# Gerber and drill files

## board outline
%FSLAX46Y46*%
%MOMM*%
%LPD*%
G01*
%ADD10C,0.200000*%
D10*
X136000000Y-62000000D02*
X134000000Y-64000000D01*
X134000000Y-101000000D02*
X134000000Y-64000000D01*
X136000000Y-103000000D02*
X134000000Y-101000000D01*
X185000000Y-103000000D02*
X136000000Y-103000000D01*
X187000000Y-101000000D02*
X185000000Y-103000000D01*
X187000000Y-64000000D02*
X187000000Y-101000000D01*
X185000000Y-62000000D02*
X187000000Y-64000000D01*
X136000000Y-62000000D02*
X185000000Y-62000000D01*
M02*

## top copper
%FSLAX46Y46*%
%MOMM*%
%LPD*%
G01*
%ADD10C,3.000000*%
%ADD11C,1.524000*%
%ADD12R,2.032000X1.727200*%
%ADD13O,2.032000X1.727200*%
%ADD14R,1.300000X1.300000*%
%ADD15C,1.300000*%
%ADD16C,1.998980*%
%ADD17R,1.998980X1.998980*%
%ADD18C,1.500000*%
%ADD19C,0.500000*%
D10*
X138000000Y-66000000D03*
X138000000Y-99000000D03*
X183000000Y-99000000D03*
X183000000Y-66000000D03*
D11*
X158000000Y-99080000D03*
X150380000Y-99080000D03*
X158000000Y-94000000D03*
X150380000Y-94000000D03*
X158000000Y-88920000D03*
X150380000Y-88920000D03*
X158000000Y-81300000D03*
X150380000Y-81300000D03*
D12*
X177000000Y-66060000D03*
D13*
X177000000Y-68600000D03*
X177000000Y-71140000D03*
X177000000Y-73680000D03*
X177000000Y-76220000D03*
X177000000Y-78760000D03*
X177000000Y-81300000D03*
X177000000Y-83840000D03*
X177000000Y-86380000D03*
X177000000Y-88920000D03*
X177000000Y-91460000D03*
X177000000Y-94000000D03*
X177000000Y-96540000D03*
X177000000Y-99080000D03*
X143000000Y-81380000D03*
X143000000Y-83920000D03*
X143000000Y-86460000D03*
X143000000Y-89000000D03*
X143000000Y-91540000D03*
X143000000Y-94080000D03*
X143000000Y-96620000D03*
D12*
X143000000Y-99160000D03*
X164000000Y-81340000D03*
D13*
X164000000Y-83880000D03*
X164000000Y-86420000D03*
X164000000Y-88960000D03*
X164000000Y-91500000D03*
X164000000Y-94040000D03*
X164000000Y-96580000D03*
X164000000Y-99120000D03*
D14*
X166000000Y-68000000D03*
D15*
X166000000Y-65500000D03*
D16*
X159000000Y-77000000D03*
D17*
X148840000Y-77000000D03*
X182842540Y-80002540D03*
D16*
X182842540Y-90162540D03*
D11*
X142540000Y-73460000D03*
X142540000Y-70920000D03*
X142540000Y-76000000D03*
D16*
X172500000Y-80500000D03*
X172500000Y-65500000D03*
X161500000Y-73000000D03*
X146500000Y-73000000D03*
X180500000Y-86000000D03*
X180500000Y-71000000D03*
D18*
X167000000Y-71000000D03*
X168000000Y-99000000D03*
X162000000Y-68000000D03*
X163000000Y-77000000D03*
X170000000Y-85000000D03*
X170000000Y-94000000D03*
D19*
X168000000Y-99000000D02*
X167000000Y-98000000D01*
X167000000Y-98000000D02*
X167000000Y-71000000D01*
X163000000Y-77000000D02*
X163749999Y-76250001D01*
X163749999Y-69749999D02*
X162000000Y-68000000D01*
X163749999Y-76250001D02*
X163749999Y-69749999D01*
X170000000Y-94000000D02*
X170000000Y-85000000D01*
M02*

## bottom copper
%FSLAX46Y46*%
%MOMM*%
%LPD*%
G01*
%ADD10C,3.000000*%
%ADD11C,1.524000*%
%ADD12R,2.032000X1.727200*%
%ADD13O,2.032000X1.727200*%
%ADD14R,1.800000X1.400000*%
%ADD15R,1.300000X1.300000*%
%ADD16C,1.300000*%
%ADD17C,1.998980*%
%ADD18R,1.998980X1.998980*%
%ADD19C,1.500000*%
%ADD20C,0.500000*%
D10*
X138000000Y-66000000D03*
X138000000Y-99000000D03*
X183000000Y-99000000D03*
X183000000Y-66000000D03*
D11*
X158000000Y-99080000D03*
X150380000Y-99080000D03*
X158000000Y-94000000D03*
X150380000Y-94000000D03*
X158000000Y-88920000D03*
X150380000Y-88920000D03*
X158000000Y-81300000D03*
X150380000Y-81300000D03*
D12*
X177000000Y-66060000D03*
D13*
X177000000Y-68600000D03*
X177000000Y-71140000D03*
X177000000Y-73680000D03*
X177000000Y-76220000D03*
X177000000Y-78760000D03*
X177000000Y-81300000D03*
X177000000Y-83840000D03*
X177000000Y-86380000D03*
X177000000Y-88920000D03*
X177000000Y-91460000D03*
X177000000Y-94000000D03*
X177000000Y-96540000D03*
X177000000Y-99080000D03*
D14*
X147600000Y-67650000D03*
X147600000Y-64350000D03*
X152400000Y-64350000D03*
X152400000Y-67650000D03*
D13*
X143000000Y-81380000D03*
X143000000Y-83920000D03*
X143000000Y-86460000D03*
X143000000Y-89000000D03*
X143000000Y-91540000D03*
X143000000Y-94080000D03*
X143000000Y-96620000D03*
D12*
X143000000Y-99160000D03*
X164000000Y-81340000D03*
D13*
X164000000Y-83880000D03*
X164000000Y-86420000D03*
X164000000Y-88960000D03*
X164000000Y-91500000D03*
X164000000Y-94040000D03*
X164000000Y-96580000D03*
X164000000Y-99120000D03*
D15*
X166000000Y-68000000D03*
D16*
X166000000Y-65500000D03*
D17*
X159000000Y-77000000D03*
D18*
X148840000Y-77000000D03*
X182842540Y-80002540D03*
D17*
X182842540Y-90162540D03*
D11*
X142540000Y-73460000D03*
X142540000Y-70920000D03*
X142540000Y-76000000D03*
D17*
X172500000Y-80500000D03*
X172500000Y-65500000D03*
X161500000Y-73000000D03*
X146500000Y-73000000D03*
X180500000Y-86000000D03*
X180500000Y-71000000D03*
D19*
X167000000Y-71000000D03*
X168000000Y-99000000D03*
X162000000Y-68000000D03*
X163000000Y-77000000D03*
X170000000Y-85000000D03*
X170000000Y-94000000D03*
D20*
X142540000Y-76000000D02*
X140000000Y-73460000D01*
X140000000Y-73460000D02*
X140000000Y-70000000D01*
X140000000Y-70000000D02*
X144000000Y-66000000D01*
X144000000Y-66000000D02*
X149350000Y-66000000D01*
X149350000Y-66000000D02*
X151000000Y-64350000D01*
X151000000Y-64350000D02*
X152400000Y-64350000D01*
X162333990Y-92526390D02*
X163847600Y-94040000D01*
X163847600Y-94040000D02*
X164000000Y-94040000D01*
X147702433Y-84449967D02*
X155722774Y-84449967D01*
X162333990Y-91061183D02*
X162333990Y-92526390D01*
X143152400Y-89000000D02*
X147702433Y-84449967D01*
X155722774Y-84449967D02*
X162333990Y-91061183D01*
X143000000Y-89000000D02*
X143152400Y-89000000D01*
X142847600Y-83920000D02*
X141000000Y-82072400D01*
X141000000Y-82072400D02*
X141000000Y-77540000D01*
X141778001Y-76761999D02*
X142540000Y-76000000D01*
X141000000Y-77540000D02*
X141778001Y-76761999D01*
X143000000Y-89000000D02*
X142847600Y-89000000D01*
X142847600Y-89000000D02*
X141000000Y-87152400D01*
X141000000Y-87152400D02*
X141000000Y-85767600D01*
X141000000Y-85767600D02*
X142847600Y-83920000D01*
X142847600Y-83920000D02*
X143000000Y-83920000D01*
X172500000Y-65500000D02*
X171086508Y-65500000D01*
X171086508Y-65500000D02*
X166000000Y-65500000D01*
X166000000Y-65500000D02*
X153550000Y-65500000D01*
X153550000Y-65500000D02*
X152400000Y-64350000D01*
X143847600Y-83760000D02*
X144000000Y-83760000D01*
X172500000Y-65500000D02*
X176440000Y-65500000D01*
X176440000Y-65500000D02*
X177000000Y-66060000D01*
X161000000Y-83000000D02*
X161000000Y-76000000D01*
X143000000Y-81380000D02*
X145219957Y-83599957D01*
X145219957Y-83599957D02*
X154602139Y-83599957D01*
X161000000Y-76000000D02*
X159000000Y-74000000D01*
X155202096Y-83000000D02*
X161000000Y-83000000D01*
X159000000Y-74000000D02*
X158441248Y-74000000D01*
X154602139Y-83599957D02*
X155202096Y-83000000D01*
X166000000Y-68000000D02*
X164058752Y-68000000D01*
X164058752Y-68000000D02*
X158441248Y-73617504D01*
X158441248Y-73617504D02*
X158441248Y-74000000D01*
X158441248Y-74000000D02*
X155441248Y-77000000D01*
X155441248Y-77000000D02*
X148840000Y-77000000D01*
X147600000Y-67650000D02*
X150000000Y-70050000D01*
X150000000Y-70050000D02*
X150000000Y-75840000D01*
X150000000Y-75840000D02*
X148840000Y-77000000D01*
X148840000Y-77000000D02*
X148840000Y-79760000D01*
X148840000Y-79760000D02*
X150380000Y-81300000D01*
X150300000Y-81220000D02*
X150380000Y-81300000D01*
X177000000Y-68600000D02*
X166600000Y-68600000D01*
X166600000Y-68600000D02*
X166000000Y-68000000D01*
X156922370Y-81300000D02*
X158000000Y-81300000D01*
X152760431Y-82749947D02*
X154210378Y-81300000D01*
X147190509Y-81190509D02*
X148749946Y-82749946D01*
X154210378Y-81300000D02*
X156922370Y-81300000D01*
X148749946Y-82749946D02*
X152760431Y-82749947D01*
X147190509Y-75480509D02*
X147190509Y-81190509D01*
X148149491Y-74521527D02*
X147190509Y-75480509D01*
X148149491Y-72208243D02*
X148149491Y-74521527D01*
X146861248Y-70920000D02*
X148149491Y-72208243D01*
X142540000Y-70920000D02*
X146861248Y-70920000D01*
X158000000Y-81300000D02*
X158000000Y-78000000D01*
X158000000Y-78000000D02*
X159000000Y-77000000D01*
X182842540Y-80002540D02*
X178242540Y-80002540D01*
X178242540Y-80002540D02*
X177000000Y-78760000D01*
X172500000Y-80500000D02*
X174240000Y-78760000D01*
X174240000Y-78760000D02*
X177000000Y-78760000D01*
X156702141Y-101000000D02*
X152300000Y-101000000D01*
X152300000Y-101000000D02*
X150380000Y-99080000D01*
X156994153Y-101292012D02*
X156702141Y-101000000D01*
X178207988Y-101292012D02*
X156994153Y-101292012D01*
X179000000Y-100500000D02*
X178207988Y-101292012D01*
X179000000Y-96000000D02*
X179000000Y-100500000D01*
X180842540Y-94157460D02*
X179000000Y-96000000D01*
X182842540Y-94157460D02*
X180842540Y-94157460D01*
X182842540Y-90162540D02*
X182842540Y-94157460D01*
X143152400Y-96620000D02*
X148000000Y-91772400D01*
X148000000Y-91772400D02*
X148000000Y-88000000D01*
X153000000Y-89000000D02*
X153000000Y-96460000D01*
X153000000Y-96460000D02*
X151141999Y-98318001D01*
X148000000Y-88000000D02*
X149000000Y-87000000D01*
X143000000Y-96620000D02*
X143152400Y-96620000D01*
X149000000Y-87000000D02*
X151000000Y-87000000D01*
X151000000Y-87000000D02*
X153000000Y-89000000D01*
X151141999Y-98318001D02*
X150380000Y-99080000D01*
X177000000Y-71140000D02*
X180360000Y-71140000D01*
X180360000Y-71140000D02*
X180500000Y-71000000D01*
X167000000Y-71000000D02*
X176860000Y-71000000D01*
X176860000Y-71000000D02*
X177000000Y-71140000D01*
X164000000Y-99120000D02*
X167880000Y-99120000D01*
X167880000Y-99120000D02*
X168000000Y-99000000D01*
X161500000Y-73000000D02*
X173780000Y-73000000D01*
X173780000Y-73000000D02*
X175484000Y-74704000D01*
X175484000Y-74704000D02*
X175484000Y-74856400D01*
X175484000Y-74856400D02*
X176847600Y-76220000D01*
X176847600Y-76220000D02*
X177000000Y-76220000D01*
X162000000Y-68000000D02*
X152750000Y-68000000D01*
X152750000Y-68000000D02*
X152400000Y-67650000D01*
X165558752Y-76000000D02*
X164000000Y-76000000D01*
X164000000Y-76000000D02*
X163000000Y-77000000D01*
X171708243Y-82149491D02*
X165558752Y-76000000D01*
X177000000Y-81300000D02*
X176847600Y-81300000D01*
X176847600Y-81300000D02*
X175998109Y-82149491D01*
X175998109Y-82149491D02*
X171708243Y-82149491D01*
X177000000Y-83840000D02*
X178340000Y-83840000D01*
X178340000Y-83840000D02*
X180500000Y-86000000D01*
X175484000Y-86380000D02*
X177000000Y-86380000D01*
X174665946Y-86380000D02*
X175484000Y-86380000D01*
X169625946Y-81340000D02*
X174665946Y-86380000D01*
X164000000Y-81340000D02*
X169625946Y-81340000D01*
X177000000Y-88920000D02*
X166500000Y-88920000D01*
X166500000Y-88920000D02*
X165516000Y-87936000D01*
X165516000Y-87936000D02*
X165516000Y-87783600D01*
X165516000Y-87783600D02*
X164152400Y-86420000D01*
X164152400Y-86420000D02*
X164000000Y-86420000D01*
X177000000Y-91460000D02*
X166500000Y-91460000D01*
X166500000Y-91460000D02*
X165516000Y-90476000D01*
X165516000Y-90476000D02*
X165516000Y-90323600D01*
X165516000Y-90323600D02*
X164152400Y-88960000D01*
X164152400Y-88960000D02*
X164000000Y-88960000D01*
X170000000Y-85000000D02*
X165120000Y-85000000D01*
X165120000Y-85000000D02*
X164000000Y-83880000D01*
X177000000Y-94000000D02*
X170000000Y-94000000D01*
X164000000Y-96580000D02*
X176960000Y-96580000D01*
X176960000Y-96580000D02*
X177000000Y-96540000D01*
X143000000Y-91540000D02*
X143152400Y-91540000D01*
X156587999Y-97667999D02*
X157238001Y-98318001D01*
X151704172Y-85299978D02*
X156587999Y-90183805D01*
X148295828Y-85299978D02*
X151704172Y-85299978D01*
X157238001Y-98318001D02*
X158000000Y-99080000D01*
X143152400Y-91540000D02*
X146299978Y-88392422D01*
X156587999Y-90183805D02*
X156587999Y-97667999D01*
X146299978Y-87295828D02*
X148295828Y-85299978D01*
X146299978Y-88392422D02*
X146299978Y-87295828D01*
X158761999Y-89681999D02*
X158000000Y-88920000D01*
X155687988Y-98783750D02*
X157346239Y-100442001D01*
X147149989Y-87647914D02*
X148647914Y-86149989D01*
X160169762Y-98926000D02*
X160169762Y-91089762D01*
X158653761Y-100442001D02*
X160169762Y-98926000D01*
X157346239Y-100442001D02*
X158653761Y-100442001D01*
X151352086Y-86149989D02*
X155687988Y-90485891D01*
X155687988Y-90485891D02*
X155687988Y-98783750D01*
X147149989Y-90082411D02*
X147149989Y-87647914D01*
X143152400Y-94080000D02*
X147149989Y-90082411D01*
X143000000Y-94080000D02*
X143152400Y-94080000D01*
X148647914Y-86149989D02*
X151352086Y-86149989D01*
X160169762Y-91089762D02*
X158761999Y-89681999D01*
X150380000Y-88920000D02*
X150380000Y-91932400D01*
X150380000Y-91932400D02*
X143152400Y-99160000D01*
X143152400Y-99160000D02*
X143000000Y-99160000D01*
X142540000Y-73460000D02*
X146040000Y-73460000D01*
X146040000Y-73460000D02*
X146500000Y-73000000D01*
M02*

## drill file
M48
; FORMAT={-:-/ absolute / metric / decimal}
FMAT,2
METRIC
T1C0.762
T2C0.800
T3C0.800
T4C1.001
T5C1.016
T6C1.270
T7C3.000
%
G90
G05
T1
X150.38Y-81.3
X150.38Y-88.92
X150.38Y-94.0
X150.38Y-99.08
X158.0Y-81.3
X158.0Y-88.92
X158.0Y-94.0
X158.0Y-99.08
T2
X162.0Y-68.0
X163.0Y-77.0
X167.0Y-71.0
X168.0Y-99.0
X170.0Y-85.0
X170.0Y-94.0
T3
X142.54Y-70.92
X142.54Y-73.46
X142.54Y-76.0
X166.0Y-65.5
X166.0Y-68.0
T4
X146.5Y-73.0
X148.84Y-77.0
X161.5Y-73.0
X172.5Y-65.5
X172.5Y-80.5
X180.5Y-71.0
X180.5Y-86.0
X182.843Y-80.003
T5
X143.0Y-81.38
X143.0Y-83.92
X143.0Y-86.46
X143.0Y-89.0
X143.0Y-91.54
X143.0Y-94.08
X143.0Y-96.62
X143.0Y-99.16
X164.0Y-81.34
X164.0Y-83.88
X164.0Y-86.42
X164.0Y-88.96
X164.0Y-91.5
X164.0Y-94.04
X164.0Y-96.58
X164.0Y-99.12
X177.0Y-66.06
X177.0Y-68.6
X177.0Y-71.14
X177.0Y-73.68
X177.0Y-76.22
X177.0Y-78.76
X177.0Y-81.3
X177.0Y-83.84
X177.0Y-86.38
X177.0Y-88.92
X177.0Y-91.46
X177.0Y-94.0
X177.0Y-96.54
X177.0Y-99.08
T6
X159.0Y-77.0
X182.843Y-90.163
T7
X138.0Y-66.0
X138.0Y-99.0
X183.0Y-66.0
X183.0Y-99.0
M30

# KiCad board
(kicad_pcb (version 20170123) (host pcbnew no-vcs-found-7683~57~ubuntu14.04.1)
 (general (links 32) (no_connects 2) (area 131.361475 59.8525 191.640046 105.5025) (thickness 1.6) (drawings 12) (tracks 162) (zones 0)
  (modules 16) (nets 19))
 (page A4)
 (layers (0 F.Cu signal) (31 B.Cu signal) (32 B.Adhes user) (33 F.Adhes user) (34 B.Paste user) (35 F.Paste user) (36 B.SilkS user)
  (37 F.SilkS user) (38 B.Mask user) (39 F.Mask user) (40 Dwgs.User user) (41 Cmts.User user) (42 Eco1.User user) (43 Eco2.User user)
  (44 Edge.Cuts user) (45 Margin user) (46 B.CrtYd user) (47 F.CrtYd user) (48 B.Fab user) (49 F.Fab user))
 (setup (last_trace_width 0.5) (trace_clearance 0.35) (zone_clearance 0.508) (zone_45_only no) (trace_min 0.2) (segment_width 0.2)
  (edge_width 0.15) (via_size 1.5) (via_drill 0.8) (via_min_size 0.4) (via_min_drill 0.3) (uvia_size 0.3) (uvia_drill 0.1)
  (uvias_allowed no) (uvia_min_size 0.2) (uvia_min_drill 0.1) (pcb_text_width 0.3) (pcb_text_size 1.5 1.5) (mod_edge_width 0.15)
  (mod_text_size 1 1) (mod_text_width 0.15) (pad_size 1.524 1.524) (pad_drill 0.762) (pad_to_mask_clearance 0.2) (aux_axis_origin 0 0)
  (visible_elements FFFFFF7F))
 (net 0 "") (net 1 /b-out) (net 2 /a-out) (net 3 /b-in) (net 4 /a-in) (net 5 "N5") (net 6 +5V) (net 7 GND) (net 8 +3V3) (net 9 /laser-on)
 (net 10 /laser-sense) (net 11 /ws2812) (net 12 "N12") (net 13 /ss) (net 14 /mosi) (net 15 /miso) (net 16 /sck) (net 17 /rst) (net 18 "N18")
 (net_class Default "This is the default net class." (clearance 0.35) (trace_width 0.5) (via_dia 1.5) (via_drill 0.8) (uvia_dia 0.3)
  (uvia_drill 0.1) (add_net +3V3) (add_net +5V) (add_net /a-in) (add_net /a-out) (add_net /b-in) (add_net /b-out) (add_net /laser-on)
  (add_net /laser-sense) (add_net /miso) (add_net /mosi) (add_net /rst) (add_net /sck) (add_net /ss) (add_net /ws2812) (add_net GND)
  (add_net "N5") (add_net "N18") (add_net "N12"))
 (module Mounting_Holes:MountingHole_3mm (layer F.Cu) (at 138 66)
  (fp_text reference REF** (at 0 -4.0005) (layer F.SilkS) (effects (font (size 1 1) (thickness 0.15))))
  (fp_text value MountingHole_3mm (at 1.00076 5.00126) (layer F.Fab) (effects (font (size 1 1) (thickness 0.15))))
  (pad 1 thru_hole circle (at 0 0) (size 3 3) (drill 3) (layers)))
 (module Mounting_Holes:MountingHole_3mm (layer F.Cu) (at 138 99)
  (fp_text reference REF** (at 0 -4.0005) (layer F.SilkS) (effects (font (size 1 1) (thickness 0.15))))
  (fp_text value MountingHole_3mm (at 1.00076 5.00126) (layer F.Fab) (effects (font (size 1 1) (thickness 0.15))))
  (pad 1 thru_hole circle (at 0 0) (size 3 3) (drill 3) (layers)))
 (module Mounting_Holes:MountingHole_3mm (layer F.Cu) (at 183 99)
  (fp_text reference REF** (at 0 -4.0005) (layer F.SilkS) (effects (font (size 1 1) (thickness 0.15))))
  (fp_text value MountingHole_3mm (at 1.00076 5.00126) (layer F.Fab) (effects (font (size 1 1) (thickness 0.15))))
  (pad 1 thru_hole circle (at 0 0) (size 3 3) (drill 3) (layers)))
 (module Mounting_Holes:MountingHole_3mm (layer F.Cu) (at 183 66)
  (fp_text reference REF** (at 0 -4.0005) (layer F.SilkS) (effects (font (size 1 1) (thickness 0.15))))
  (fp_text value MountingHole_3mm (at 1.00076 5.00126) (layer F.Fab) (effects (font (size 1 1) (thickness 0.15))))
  (pad 1 thru_hole circle (at 0 0) (size 3 3) (drill 3) (layers)))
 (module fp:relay (layer F.Cu) (at 154.19 81.3)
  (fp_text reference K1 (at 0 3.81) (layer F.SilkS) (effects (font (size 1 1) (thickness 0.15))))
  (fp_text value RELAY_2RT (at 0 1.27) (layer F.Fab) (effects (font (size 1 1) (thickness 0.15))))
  (pad 1 thru_hole circle (at 3.81 17.78) (size 1.524 1.524) (drill 0.762) (layers *.Cu *.Mask) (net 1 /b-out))
  (pad 16 thru_hole circle (at -3.81 17.78) (size 1.524 1.524) (drill 0.762) (layers *.Cu *.Mask) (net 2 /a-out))
  (pad 3 thru_hole circle (at 3.81 12.7) (size 1.524 1.524) (drill 0.762) (layers *.Cu *.Mask))
  (pad 14 thru_hole circle (at -3.81 12.7) (size 1.524 1.524) (drill 0.762) (layers *.Cu *.Mask))
  (pad 5 thru_hole circle (at 3.81 7.62) (size 1.524 1.524) (drill 0.762) (layers *.Cu *.Mask) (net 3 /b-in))
  (pad 12 thru_hole circle (at -3.81 7.62) (size 1.524 1.524) (drill 0.762) (layers *.Cu *.Mask) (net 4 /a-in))
  (pad 9 thru_hole circle (at 3.81 0) (size 1.524 1.524) (drill 0.762) (layers *.Cu *.Mask) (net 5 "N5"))
  (pad 8 thru_hole circle (at -3.81 0) (size 1.524 1.524) (drill 0.762) (layers *.Cu *.Mask) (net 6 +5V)))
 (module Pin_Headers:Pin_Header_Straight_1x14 (layer F.Cu) (at 177 66.06)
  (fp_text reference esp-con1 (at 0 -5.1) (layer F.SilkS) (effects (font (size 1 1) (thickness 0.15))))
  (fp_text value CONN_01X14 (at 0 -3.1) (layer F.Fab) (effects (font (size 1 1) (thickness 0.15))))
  (pad 1 thru_hole rect (at 0 0) (size 2.032 1.7272) (drill 1.016) (layers *.Cu *.Mask F.SilkS) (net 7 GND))
  (pad 2 thru_hole oval (at 0 2.54) (size 2.032 1.7272) (drill 1.016) (layers *.Cu *.Mask F.SilkS) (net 6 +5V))
  (pad 3 thru_hole oval (at 0 5.08) (size 2.032 1.7272) (drill 1.016) (layers *.Cu *.Mask F.SilkS) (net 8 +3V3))
  (pad 4 thru_hole oval (at 0 7.62) (size 2.032 1.7272) (drill 1.016) (layers *.Cu *.Mask F.SilkS))
  (pad 5 thru_hole oval (at 0 10.16) (size 2.032 1.7272) (drill 1.016) (layers *.Cu *.Mask F.SilkS) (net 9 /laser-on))
  (pad 6 thru_hole oval (at 0 12.7) (size 2.032 1.7272) (drill 1.016) (layers *.Cu *.Mask F.SilkS) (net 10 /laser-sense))
  (pad 7 thru_hole oval (at 0 15.24) (size 2.032 1.7272) (drill 1.016) (layers *.Cu *.Mask F.SilkS) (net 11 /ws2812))
  (pad 8 thru_hole oval (at 0 17.78) (size 2.032 1.7272) (drill 1.016) (layers *.Cu *.Mask F.SilkS) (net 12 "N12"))
  (pad 9 thru_hole oval (at 0 20.32) (size 2.032 1.7272) (drill 1.016) (layers *.Cu *.Mask F.SilkS) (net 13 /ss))
  (pad 10 thru_hole oval (at 0 22.86) (size 2.032 1.7272) (drill 1.016) (layers *.Cu *.Mask F.SilkS) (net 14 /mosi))
  (pad 11 thru_hole oval (at 0 25.4) (size 2.032 1.7272) (drill 1.016) (layers *.Cu *.Mask F.SilkS) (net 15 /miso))
  (pad 12 thru_hole oval (at 0 27.94) (size 2.032 1.7272) (drill 1.016) (layers *.Cu *.Mask F.SilkS) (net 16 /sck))
  (pad 13 thru_hole oval (at 0 30.48) (size 2.032 1.7272) (drill 1.016) (layers *.Cu *.Mask F.SilkS) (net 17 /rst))
  (pad 14 thru_hole oval (at 0 33.02) (size 2.032 1.7272) (drill 1.016) (layers *.Cu *.Mask F.SilkS)))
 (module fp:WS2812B (layer B.Cu) (at 150 66 270)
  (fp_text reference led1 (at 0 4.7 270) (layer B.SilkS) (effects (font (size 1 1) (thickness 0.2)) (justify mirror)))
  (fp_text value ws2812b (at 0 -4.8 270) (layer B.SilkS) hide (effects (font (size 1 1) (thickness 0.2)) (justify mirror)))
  (pad 1 smd rect (at 1.65 2.4 270) (size 1.4 1.8) (layers B.Cu B.Paste B.Mask) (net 6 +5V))
  (pad 2 smd rect (at -1.65 2.4 270) (size 1.4 1.8) (layers B.Cu B.Paste B.Mask))
  (pad 3 smd rect (at -1.65 -2.4 270) (size 1.4 1.8) (layers B.Cu B.Paste B.Mask) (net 7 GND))
  (pad 4 smd rect (at 1.65 -2.4 270) (size 1.4 1.8) (layers B.Cu B.Paste B.Mask) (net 11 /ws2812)))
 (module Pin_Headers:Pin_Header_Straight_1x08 (layer F.Cu) (at 143 99.16 180)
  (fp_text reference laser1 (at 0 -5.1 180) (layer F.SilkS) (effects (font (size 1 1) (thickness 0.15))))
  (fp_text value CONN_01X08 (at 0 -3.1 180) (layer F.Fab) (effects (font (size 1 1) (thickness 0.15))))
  (pad 8 thru_hole oval (at 0 17.78 180) (size 2.032 1.7272) (drill 1.016) (layers *.Cu *.Mask F.SilkS) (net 6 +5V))
  (pad 7 thru_hole oval (at 0 15.24 180) (size 2.032 1.7272) (drill 1.016) (layers *.Cu *.Mask F.SilkS) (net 7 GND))
  (pad 6 thru_hole oval (at 0 12.7 180) (size 2.032 1.7272) (drill 1.016) (layers *.Cu *.Mask F.SilkS))
  (pad 5 thru_hole oval (at 0 10.16 180) (size 2.032 1.7272) (drill 1.016) (layers *.Cu *.Mask F.SilkS) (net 7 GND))
  (pad 4 thru_hole oval (at 0 7.62 180) (size 2.032 1.7272) (drill 1.016) (layers *.Cu *.Mask F.SilkS) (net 1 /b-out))
  (pad 3 thru_hole oval (at 0 5.08 180) (size 2.032 1.7272) (drill 1.016) (layers *.Cu *.Mask F.SilkS) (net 3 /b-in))
  (pad 2 thru_hole oval (at 0 2.54 180) (size 2.032 1.7272) (drill 1.016) (layers *.Cu *.Mask F.SilkS) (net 2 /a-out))
  (pad 1 thru_hole rect (at 0 0 180) (size 2.032 1.7272) (drill 1.016) (layers *.Cu *.Mask F.SilkS) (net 4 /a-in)))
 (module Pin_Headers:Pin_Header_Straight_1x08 (layer F.Cu) (at 164 81.34)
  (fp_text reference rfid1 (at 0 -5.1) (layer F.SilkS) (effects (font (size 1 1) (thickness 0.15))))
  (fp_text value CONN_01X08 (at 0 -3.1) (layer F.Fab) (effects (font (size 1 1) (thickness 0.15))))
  (pad 1 thru_hole rect (at 0 0) (size 2.032 1.7272) (drill 1.016) (layers *.Cu *.Mask F.SilkS) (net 13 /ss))
  (pad 2 thru_hole oval (at 0 2.54) (size 2.032 1.7272) (drill 1.016) (layers *.Cu *.Mask F.SilkS) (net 16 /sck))
  (pad 3 thru_hole oval (at 0 5.08) (size 2.032 1.7272) (drill 1.016) (layers *.Cu *.Mask F.SilkS) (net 14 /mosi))
  (pad 4 thru_hole oval (at 0 7.62) (size 2.032 1.7272) (drill 1.016) (layers *.Cu *.Mask F.SilkS) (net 15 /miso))
  (pad 5 thru_hole oval (at 0 10.16) (size 2.032 1.7272) (drill 1.016) (layers *.Cu *.Mask F.SilkS))
  (pad 6 thru_hole oval (at 0 12.7) (size 2.032 1.7272) (drill 1.016) (layers *.Cu *.Mask F.SilkS) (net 7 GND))
  (pad 7 thru_hole oval (at 0 15.24) (size 2.032 1.7272) (drill 1.016) (layers *.Cu *.Mask F.SilkS) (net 17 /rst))
  (pad 8 thru_hole oval (at 0 17.78) (size 2.032 1.7272) (drill 1.016) (layers *.Cu *.Mask F.SilkS) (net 8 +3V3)))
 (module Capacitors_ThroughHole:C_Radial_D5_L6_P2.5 (layer F.Cu) (at 166 68 90)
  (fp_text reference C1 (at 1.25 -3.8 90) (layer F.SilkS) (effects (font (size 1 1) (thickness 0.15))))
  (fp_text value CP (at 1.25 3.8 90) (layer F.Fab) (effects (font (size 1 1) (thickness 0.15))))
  (pad 1 thru_hole rect (at 0 0 90) (size 1.3 1.3) (drill 0.8) (layers *.Cu *.Mask F.SilkS) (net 6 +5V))
  (pad 2 thru_hole circle (at 2.5 0 90) (size 1.3 1.3) (drill 0.8) (layers *.Cu *.Mask F.SilkS) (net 7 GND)))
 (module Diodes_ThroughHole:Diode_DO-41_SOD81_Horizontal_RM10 (layer F.Cu) (at 148.84 77.00254)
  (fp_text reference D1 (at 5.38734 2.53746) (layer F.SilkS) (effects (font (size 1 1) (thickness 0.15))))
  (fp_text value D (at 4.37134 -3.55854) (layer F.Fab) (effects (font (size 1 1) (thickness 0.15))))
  (pad 2 thru_hole circle (at 10.16 -0.00254 180) (size 1.99898 1.99898) (drill 1.27) (layers *.Cu *.Mask F.SilkS) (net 5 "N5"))
  (pad 1 thru_hole rect (at 0 -0.00254 180) (size 1.99898 1.99898) (drill 1.00076) (layers *.Cu *.Mask F.SilkS) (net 6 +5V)))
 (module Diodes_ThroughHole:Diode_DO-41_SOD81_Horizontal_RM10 (layer F.Cu) (at 182.84 80.00254 270)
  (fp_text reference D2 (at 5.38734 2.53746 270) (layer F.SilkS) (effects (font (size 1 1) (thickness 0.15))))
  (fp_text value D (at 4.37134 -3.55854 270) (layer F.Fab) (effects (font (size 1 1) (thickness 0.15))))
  (pad 1 thru_hole rect (at 0 -0.00254 90) (size 1.99898 1.99898) (drill 1.00076) (layers *.Cu *.Mask F.SilkS) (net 10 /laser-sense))
  (pad 2 thru_hole circle (at 10.16 -0.00254 90) (size 1.99898 1.99898) (drill 1.27) (layers *.Cu *.Mask F.SilkS) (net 2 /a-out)))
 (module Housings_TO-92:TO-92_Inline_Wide (layer F.Cu) (at 142.54 76 90)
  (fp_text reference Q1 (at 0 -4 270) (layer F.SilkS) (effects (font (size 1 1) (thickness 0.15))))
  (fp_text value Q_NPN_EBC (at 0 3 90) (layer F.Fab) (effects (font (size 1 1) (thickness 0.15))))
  (pad 2 thru_hole circle (at 2.54 0 180) (size 1.524 1.524) (drill 0.8) (layers *.Cu *.Mask F.SilkS) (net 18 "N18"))
  (pad 3 thru_hole circle (at 5.08 0 180) (size 1.524 1.524) (drill 0.8) (layers *.Cu *.Mask F.SilkS) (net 5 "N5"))
  (pad 1 thru_hole circle (at 0 0 180) (size 1.524 1.524) (drill 0.8) (layers *.Cu *.Mask F.SilkS) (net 7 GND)))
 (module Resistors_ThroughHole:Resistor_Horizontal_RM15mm (layer F.Cu) (at 172.5 73 90)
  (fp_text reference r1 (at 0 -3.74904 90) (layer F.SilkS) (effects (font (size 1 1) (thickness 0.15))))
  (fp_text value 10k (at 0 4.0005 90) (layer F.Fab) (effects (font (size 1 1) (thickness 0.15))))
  (pad 1 thru_hole circle (at -7.5 0 90) (size 1.99898 1.99898) (drill 1.00076) (layers *.Cu *.SilkS *.Mask) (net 10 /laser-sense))
  (pad 2 thru_hole circle (at 7.5 0 90) (size 1.99898 1.99898) (drill 1.00076) (layers *.Cu *.SilkS *.Mask) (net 7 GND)))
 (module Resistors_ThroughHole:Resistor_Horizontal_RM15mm (layer F.Cu) (at 154 73)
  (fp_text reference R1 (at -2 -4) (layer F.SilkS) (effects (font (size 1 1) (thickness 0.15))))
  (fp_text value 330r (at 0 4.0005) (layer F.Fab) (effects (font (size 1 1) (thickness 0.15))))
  (pad 2 thru_hole circle (at 7.5 0) (size 1.99898 1.99898) (drill 1.00076) (layers *.Cu *.SilkS *.Mask) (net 9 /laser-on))
  (pad 1 thru_hole circle (at -7.5 0) (size 1.99898 1.99898) (drill 1.00076) (layers *.Cu *.SilkS *.Mask) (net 18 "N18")))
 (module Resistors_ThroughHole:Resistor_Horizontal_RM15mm (layer F.Cu) (at 180.5 78.5 90)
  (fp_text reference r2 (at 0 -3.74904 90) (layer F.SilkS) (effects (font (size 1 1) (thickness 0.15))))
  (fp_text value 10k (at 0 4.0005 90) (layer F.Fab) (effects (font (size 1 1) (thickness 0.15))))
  (pad 1 thru_hole circle (at -7.5 0 90) (size 1.99898 1.99898) (drill 1.00076) (layers *.Cu *.SilkS *.Mask) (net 12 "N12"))
  (pad 2 thru_hole circle (at 7.5 0 90) (size 1.99898 1.99898) (drill 1.00076) (layers *.Cu *.SilkS *.Mask) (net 8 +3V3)))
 (gr_line (start 136 62) (end 134 64) (layer Edge.Cuts) (width 0.2))
 (gr_line (start 134 101) (end 134 64) (layer Edge.Cuts) (width 0.2))
 (gr_line (start 136 103) (end 134 101) (layer Edge.Cuts) (width 0.2))
 (gr_line (start 185 103) (end 136 103) (layer Edge.Cuts) (width 0.2))
 (gr_line (start 187 101) (end 185 103) (layer Edge.Cuts) (width 0.2))
 (gr_line (start 187 64) (end 187 101) (layer Edge.Cuts) (width 0.2))
 (gr_line (start 185 62) (end 187 64) (layer Edge.Cuts) (width 0.2))
 (gr_line (start 136 62) (end 185 62) (layer Edge.Cuts) (width 0.2))
 (segment (start 142.54 76) (end 140 73.46) (width 0.5) (layer B.Cu) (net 7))
 (segment (start 140 73.46) (end 140 70) (width 0.5) (layer B.Cu) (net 7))
 (segment (start 140 70) (end 144 66) (width 0.5) (layer B.Cu) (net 7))
 (segment (start 144 66) (end 149.35 66) (width 0.5) (layer B.Cu) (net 7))
 (segment (start 149.35 66) (end 151 64.35) (width 0.5) (layer B.Cu) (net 7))
 (segment (start 151 64.35) (end 152.4 64.35) (width 0.5) (layer B.Cu) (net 7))
 (segment (start 162.33399 92.52639) (end 163.8476 94.04) (width 0.5) (layer B.Cu) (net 7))
 (segment (start 163.8476 94.04) (end 164 94.04) (width 0.5) (layer B.Cu) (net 7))
 (segment (start 147.702433 84.449967) (end 155.722774 84.449967) (width 0.5) (layer B.Cu) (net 7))
 (segment (start 162.33399 91.061183) (end 162.33399 92.52639) (width 0.5) (layer B.Cu) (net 7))
 (segment (start 143.1524 89) (end 147.702433 84.449967) (width 0.5) (layer B.Cu) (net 7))
 (segment (start 155.722774 84.449967) (end 162.33399 91.061183) (width 0.5) (layer B.Cu) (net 7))
 (segment (start 143 89) (end 143.1524 89) (width 0.5) (layer B.Cu) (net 7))
 (segment (start 142.8476 83.92) (end 141 82.0724) (width 0.5) (layer B.Cu) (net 7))
 (segment (start 141 82.0724) (end 141 77.54) (width 0.5) (layer B.Cu) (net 7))
 (segment (start 141.778001 76.761999) (end 142.54 76) (width 0.5) (layer B.Cu) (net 7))
 (segment (start 141 77.54) (end 141.778001 76.761999) (width 0.5) (layer B.Cu) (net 7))
 (segment (start 143 89) (end 142.8476 89) (width 0.5) (layer B.Cu) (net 7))
 (segment (start 142.8476 89) (end 141 87.1524) (width 0.5) (layer B.Cu) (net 7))
 (segment (start 141 87.1524) (end 141 85.7676) (width 0.5) (layer B.Cu) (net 7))
 (segment (start 141 85.7676) (end 142.8476 83.92) (width 0.5) (layer B.Cu) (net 7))
 (segment (start 142.8476 83.92) (end 143 83.92) (width 0.5) (layer B.Cu) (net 7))
 (segment (start 172.5 65.5) (end 171.086508 65.5) (width 0.5) (layer B.Cu) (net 7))
 (segment (start 171.086508 65.5) (end 166 65.5) (width 0.5) (layer B.Cu) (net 7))
 (segment (start 166 65.5) (end 153.55 65.5) (width 0.5) (layer B.Cu) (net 7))
 (segment (start 153.55 65.5) (end 152.4 64.35) (width 0.5) (layer B.Cu) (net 7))
 (segment (start 143.8476 83.76) (end 144 83.76) (width 0.5) (layer B.Cu) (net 7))
 (segment (start 172.5 65.5) (end 176.44 65.5) (width 0.5) (layer B.Cu) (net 7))
 (segment (start 176.44 65.5) (end 177 66.06) (width 0.5) (layer B.Cu) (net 7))
 (segment (start 161 83) (end 161 76) (width 0.5) (layer B.Cu) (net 6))
 (segment (start 143 81.38) (end 145.219957 83.599957) (width 0.5) (layer B.Cu) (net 6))
 (segment (start 145.219957 83.599957) (end 154.602139 83.599957) (width 0.5) (layer B.Cu) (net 6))
 (segment (start 161 76) (end 159 74) (width 0.5) (layer B.Cu) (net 6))
 (segment (start 155.202096 83) (end 161 83) (width 0.5) (layer B.Cu) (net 6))
 (segment (start 159 74) (end 158.441248 74) (width 0.5) (layer B.Cu) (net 6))
 (segment (start 154.602139 83.599957) (end 155.202096 83) (width 0.5) (layer B.Cu) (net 6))
 (segment (start 166 68) (end 164.058752 68) (width 0.5) (layer B.Cu) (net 6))
 (segment (start 164.058752 68) (end 158.441248 73.617504) (width 0.5) (layer B.Cu) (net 6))
 (segment (start 158.441248 73.617504) (end 158.441248 74) (width 0.5) (layer B.Cu) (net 6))
 (segment (start 158.441248 74) (end 155.441248 77) (width 0.5) (layer B.Cu) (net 6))
 (segment (start 155.441248 77) (end 148.84 77) (width 0.5) (layer B.Cu) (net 6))
 (segment (start 147.6 67.65) (end 150 70.05) (width 0.5) (layer B.Cu) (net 6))
 (segment (start 150 70.05) (end 150 75.84) (width 0.5) (layer B.Cu) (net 6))
 (segment (start 150 75.84) (end 148.84 77) (width 0.5) (layer B.Cu) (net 6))
 (segment (start 148.84 77) (end 148.84 79.76) (width 0.5) (layer B.Cu) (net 6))
 (segment (start 148.84 79.76) (end 150.38 81.3) (width 0.5) (layer B.Cu) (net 6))
 (segment (start 150.3 81.22) (end 150.38 81.3) (width 0.5) (layer B.Cu) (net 6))
 (segment (start 177 68.6) (end 166.6 68.6) (width 0.5) (layer B.Cu) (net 6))
 (segment (start 166.6 68.6) (end 166 68) (width 0.5) (layer B.Cu) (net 6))
 (segment (start 156.92237 81.3) (end 158 81.3) (width 0.5) (layer B.Cu) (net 5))
 (segment (start 152.760431 82.749947) (end 154.210378 81.3) (width 0.5) (layer B.Cu) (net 5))
 (segment (start 147.190509 81.190509) (end 148.749946 82.749946) (width 0.5) (layer B.Cu) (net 5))
 (segment (start 154.210378 81.3) (end 156.92237 81.3) (width 0.5) (layer B.Cu) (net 5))
 (segment (start 148.749946 82.749946) (end 152.760431 82.749947) (width 0.5) (layer B.Cu) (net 5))
 (segment (start 147.190509 75.480509) (end 147.190509 81.190509) (width 0.5) (layer B.Cu) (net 5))
 (segment (start 148.149491 74.521527) (end 147.190509 75.480509) (width 0.5) (layer B.Cu) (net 5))
 (segment (start 148.149491 72.208243) (end 148.149491 74.521527) (width 0.5) (layer B.Cu) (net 5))
 (segment (start 146.861248 70.92) (end 148.149491 72.208243) (width 0.5) (layer B.Cu) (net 5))
 (segment (start 142.54 70.92) (end 146.861248 70.92) (width 0.5) (layer B.Cu) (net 5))
 (segment (start 158 81.3) (end 158 78) (width 0.5) (layer B.Cu) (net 5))
 (segment (start 158 78) (end 159 77) (width 0.5) (layer B.Cu) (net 5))
 (segment (start 182.84254 80.00254) (end 178.24254 80.00254) (width 0.5) (layer B.Cu) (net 10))
 (segment (start 178.24254 80.00254) (end 177 78.76) (width 0.5) (layer B.Cu) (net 10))
 (segment (start 172.5 80.5) (end 174.24 78.76) (width 0.5) (layer B.Cu) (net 10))
 (segment (start 174.24 78.76) (end 177 78.76) (width 0.5) (layer B.Cu) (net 10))
 (segment (start 156.702141 101) (end 152.3 101) (width 0.5) (layer B.Cu) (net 2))
 (segment (start 152.3 101) (end 150.38 99.08) (width 0.5) (layer B.Cu) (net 2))
 (segment (start 156.994153 101.292012) (end 156.702141 101) (width 0.5) (layer B.Cu) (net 2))
 (segment (start 178.207988 101.292012) (end 156.994153 101.292012) (width 0.5) (layer B.Cu) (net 2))
 (segment (start 179 100.5) (end 178.207988 101.292012) (width 0.5) (layer B.Cu) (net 2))
 (segment (start 179 96) (end 179 100.5) (width 0.5) (layer B.Cu) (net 2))
 (segment (start 180.84254 94.15746) (end 179 96) (width 0.5) (layer B.Cu) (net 2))
 (segment (start 182.84254 94.15746) (end 180.84254 94.15746) (width 0.5) (layer B.Cu) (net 2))
 (segment (start 182.84254 90.16254) (end 182.84254 94.15746) (width 0.5) (layer B.Cu) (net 2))
 (segment (start 143.1524 96.62) (end 148 91.7724) (width 0.5) (layer B.Cu) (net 2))
 (segment (start 148 91.7724) (end 148 88) (width 0.5) (layer B.Cu) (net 2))
 (segment (start 153 89) (end 153 96.46) (width 0.5) (layer B.Cu) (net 2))
 (segment (start 153 96.46) (end 151.141999 98.318001) (width 0.5) (layer B.Cu) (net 2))
 (segment (start 148 88) (end 149 87) (width 0.5) (layer B.Cu) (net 2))
 (segment (start 143 96.62) (end 143.1524 96.62) (width 0.5) (layer B.Cu) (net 2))
 (segment (start 149 87) (end 151 87) (width 0.5) (layer B.Cu) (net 2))
 (segment (start 151 87) (end 153 89) (width 0.5) (layer B.Cu) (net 2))
 (segment (start 151.141999 98.318001) (end 150.38 99.08) (width 0.5) (layer B.Cu) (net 2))
 (segment (start 177 71.14) (end 180.36 71.14) (width 0.5) (layer B.Cu) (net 8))
 (segment (start 180.36 71.14) (end 180.5 71) (width 0.5) (layer B.Cu) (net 8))
 (segment (start 167 71) (end 176.86 71) (width 0.5) (layer B.Cu) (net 8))
 (segment (start 176.86 71) (end 177 71.14) (width 0.5) (layer B.Cu) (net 8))
 (segment (start 168 99) (end 167 98) (width 0.5) (layer F.Cu) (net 8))
 (segment (start 167 98) (end 167 71) (width 0.5) (layer F.Cu) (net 8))
 (via (at 167 71) (size 1.5) (drill 0.8) (layers F.Cu B.Cu) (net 8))
 (segment (start 164 99.12) (end 167.88 99.12) (width 0.5) (layer B.Cu) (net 8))
 (via (at 168 99) (size 1.5) (drill 0.8) (layers F.Cu B.Cu) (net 8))
 (segment (start 167.88 99.12) (end 168 99) (width 0.5) (layer B.Cu) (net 8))
 (segment (start 161.5 73) (end 173.78 73) (width 0.5) (layer B.Cu) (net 9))
 (segment (start 173.78 73) (end 175.484 74.704) (width 0.5) (layer B.Cu) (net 9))
 (segment (start 175.484 74.704) (end 175.484 74.8564) (width 0.5) (layer B.Cu) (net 9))
 (segment (start 175.484 74.8564) (end 176.8476 76.22) (width 0.5) (layer B.Cu) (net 9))
 (segment (start 176.8476 76.22) (end 177 76.22) (width 0.5) (layer B.Cu) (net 9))
 (segment (start 162 68) (end 152.75 68) (width 0.5) (layer B.Cu) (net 11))
 (segment (start 152.75 68) (end 152.4 67.65) (width 0.5) (layer B.Cu) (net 11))
 (segment (start 163 77) (end 163.749999 76.250001) (width 0.5) (layer F.Cu) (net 11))
 (segment (start 163.749999 69.749999) (end 162 68) (width 0.5) (layer F.Cu) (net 11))
 (segment (start 163.749999 76.250001) (end 163.749999 69.749999) (width 0.5) (layer F.Cu) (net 11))
 (via (at 162 68) (size 1.5) (drill 0.8) (layers F.Cu B.Cu) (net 11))
 (segment (start 165.558752 76) (end 164 76) (width 0.5) (layer B.Cu) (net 11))
 (segment (start 164 76) (end 163 77) (width 0.5) (layer B.Cu) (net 11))
 (via (at 163 77) (size 1.5) (drill 0.8) (layers F.Cu B.Cu) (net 11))
 (segment (start 171.708243 82.149491) (end 165.558752 76) (width 0.5) (layer B.Cu) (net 11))
 (segment (start 177 81.3) (end 176.8476 81.3) (width 0.5) (layer B.Cu) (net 11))
 (segment (start 176.8476 81.3) (end 175.998109 82.149491) (width 0.5) (layer B.Cu) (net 11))
 (segment (start 175.998109 82.149491) (end 171.708243 82.149491) (width 0.5) (layer B.Cu) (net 11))
 (segment (start 177 83.84) (end 178.34 83.84) (width 0.5) (layer B.Cu) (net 12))
 (segment (start 178.34 83.84) (end 180.5 86) (width 0.5) (layer B.Cu) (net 12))
 (segment (start 175.484 86.38) (end 177 86.38) (width 0.5) (layer B.Cu) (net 13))
 (segment (start 174.665946 86.38) (end 175.484 86.38) (width 0.5) (layer B.Cu) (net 13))
 (segment (start 169.625946 81.34) (end 174.665946 86.38) (width 0.5) (layer B.Cu) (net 13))
 (segment (start 164 81.34) (end 169.625946 81.34) (width 0.5) (layer B.Cu) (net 13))
 (segment (start 177 88.92) (end 166.5 88.92) (width 0.5) (layer B.Cu) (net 14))
 (segment (start 166.5 88.92) (end 165.516 87.936) (width 0.5) (layer B.Cu) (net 14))
 (segment (start 165.516 87.936) (end 165.516 87.7836) (width 0.5) (layer B.Cu) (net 14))
 (segment (start 165.516 87.7836) (end 164.1524 86.42) (width 0.5) (layer B.Cu) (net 14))
 (segment (start 164.1524 86.42) (end 164 86.42) (width 0.5) (layer B.Cu) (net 14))
 (segment (start 177 91.46) (end 166.5 91.46) (width 0.5) (layer B.Cu) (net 15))
 (segment (start 166.5 91.46) (end 165.516 90.476) (width 0.5) (layer B.Cu) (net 15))
 (segment (start 165.516 90.476) (end 165.516 90.3236) (width 0.5) (layer B.Cu) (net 15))
 (segment (start 165.516 90.3236) (end 164.1524 88.96) (width 0.5) (layer B.Cu) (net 15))
 (segment (start 164.1524 88.96) (end 164 88.96) (width 0.5) (layer B.Cu) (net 15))
 (segment (start 170 85) (end 165.12 85) (width 0.5) (layer B.Cu) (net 16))
 (segment (start 165.12 85) (end 164 83.88) (width 0.5) (layer B.Cu) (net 16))
 (via (at 170 85) (size 1.5) (drill 0.8) (layers F.Cu B.Cu) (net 16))
 (segment (start 170 94) (end 170 85) (width 0.5) (layer F.Cu) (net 16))
 (segment (start 177 94) (end 170 94) (width 0.5) (layer B.Cu) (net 16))
 (via (at 170 94) (size 1.5) (drill 0.8) (layers F.Cu B.Cu) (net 16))
 (segment (start 164 96.58) (end 176.96 96.58) (width 0.5) (layer B.Cu) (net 17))
 (segment (start 176.96 96.58) (end 177 96.54) (width 0.5) (layer B.Cu) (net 17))
 (segment (start 143 91.54) (end 143.1524 91.54) (width 0.5) (layer B.Cu) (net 1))
 (segment (start 156.587999 97.667999) (end 157.238001 98.318001) (width 0.5) (layer B.Cu) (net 1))
 (segment (start 151.704172 85.299978) (end 156.587999 90.183805) (width 0.5) (layer B.Cu) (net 1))
 (segment (start 148.295828 85.299978) (end 151.704172 85.299978) (width 0.5) (layer B.Cu) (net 1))
 (segment (start 157.238001 98.318001) (end 158 99.08) (width 0.5) (layer B.Cu) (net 1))
 (segment (start 143.1524 91.54) (end 146.299978 88.392422) (width 0.5) (layer B.Cu) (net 1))
 (segment (start 156.587999 90.183805) (end 156.587999 97.667999) (width 0.5) (layer B.Cu) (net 1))
 (segment (start 146.299978 87.295828) (end 148.295828 85.299978) (width 0.5) (layer B.Cu) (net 1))
 (segment (start 146.299978 88.392422) (end 146.299978 87.295828) (width 0.5) (layer B.Cu) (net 1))
 (segment (start 158.761999 89.681999) (end 158 88.92) (width 0.5) (layer B.Cu) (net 3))
 (segment (start 155.687988 98.78375) (end 157.346239 100.442001) (width 0.5) (layer B.Cu) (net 3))
 (segment (start 147.149989 87.647914) (end 148.647914 86.149989) (width 0.5) (layer B.Cu) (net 3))
 (segment (start 160.169762 98.926) (end 160.169762 91.089762) (width 0.5) (layer B.Cu) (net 3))
 (segment (start 158.653761 100.442001) (end 160.169762 98.926) (width 0.5) (layer B.Cu) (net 3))
 (segment (start 157.346239 100.442001) (end 158.653761 100.442001) (width 0.5) (layer B.Cu) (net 3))
 (segment (start 151.352086 86.149989) (end 155.687988 90.485891) (width 0.5) (layer B.Cu) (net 3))
 (segment (start 155.687988 90.485891) (end 155.687988 98.78375) (width 0.5) (layer B.Cu) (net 3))
 (segment (start 147.149989 90.082411) (end 147.149989 87.647914) (width 0.5) (layer B.Cu) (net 3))
 (segment (start 143.1524 94.08) (end 147.149989 90.082411) (width 0.5) (layer B.Cu) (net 3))
 (segment (start 143 94.08) (end 143.1524 94.08) (width 0.5) (layer B.Cu) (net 3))
 (segment (start 148.647914 86.149989) (end 151.352086 86.149989) (width 0.5) (layer B.Cu) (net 3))
 (segment (start 160.169762 91.089762) (end 158.761999 89.681999) (width 0.5) (layer B.Cu) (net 3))
 (segment (start 150.38 88.92) (end 150.38 91.9324) (width 0.5) (layer B.Cu) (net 4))
 (segment (start 150.38 91.9324) (end 143.1524 99.16) (width 0.5) (layer B.Cu) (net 4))
 (segment (start 143.1524 99.16) (end 143 99.16) (width 0.5) (layer B.Cu) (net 4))
 (segment (start 142.54 73.46) (end 146.04 73.46) (width 0.5) (layer B.Cu) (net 18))
 (segment (start 146.04 73.46) (end 146.5 73) (width 0.5) (layer B.Cu) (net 18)))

